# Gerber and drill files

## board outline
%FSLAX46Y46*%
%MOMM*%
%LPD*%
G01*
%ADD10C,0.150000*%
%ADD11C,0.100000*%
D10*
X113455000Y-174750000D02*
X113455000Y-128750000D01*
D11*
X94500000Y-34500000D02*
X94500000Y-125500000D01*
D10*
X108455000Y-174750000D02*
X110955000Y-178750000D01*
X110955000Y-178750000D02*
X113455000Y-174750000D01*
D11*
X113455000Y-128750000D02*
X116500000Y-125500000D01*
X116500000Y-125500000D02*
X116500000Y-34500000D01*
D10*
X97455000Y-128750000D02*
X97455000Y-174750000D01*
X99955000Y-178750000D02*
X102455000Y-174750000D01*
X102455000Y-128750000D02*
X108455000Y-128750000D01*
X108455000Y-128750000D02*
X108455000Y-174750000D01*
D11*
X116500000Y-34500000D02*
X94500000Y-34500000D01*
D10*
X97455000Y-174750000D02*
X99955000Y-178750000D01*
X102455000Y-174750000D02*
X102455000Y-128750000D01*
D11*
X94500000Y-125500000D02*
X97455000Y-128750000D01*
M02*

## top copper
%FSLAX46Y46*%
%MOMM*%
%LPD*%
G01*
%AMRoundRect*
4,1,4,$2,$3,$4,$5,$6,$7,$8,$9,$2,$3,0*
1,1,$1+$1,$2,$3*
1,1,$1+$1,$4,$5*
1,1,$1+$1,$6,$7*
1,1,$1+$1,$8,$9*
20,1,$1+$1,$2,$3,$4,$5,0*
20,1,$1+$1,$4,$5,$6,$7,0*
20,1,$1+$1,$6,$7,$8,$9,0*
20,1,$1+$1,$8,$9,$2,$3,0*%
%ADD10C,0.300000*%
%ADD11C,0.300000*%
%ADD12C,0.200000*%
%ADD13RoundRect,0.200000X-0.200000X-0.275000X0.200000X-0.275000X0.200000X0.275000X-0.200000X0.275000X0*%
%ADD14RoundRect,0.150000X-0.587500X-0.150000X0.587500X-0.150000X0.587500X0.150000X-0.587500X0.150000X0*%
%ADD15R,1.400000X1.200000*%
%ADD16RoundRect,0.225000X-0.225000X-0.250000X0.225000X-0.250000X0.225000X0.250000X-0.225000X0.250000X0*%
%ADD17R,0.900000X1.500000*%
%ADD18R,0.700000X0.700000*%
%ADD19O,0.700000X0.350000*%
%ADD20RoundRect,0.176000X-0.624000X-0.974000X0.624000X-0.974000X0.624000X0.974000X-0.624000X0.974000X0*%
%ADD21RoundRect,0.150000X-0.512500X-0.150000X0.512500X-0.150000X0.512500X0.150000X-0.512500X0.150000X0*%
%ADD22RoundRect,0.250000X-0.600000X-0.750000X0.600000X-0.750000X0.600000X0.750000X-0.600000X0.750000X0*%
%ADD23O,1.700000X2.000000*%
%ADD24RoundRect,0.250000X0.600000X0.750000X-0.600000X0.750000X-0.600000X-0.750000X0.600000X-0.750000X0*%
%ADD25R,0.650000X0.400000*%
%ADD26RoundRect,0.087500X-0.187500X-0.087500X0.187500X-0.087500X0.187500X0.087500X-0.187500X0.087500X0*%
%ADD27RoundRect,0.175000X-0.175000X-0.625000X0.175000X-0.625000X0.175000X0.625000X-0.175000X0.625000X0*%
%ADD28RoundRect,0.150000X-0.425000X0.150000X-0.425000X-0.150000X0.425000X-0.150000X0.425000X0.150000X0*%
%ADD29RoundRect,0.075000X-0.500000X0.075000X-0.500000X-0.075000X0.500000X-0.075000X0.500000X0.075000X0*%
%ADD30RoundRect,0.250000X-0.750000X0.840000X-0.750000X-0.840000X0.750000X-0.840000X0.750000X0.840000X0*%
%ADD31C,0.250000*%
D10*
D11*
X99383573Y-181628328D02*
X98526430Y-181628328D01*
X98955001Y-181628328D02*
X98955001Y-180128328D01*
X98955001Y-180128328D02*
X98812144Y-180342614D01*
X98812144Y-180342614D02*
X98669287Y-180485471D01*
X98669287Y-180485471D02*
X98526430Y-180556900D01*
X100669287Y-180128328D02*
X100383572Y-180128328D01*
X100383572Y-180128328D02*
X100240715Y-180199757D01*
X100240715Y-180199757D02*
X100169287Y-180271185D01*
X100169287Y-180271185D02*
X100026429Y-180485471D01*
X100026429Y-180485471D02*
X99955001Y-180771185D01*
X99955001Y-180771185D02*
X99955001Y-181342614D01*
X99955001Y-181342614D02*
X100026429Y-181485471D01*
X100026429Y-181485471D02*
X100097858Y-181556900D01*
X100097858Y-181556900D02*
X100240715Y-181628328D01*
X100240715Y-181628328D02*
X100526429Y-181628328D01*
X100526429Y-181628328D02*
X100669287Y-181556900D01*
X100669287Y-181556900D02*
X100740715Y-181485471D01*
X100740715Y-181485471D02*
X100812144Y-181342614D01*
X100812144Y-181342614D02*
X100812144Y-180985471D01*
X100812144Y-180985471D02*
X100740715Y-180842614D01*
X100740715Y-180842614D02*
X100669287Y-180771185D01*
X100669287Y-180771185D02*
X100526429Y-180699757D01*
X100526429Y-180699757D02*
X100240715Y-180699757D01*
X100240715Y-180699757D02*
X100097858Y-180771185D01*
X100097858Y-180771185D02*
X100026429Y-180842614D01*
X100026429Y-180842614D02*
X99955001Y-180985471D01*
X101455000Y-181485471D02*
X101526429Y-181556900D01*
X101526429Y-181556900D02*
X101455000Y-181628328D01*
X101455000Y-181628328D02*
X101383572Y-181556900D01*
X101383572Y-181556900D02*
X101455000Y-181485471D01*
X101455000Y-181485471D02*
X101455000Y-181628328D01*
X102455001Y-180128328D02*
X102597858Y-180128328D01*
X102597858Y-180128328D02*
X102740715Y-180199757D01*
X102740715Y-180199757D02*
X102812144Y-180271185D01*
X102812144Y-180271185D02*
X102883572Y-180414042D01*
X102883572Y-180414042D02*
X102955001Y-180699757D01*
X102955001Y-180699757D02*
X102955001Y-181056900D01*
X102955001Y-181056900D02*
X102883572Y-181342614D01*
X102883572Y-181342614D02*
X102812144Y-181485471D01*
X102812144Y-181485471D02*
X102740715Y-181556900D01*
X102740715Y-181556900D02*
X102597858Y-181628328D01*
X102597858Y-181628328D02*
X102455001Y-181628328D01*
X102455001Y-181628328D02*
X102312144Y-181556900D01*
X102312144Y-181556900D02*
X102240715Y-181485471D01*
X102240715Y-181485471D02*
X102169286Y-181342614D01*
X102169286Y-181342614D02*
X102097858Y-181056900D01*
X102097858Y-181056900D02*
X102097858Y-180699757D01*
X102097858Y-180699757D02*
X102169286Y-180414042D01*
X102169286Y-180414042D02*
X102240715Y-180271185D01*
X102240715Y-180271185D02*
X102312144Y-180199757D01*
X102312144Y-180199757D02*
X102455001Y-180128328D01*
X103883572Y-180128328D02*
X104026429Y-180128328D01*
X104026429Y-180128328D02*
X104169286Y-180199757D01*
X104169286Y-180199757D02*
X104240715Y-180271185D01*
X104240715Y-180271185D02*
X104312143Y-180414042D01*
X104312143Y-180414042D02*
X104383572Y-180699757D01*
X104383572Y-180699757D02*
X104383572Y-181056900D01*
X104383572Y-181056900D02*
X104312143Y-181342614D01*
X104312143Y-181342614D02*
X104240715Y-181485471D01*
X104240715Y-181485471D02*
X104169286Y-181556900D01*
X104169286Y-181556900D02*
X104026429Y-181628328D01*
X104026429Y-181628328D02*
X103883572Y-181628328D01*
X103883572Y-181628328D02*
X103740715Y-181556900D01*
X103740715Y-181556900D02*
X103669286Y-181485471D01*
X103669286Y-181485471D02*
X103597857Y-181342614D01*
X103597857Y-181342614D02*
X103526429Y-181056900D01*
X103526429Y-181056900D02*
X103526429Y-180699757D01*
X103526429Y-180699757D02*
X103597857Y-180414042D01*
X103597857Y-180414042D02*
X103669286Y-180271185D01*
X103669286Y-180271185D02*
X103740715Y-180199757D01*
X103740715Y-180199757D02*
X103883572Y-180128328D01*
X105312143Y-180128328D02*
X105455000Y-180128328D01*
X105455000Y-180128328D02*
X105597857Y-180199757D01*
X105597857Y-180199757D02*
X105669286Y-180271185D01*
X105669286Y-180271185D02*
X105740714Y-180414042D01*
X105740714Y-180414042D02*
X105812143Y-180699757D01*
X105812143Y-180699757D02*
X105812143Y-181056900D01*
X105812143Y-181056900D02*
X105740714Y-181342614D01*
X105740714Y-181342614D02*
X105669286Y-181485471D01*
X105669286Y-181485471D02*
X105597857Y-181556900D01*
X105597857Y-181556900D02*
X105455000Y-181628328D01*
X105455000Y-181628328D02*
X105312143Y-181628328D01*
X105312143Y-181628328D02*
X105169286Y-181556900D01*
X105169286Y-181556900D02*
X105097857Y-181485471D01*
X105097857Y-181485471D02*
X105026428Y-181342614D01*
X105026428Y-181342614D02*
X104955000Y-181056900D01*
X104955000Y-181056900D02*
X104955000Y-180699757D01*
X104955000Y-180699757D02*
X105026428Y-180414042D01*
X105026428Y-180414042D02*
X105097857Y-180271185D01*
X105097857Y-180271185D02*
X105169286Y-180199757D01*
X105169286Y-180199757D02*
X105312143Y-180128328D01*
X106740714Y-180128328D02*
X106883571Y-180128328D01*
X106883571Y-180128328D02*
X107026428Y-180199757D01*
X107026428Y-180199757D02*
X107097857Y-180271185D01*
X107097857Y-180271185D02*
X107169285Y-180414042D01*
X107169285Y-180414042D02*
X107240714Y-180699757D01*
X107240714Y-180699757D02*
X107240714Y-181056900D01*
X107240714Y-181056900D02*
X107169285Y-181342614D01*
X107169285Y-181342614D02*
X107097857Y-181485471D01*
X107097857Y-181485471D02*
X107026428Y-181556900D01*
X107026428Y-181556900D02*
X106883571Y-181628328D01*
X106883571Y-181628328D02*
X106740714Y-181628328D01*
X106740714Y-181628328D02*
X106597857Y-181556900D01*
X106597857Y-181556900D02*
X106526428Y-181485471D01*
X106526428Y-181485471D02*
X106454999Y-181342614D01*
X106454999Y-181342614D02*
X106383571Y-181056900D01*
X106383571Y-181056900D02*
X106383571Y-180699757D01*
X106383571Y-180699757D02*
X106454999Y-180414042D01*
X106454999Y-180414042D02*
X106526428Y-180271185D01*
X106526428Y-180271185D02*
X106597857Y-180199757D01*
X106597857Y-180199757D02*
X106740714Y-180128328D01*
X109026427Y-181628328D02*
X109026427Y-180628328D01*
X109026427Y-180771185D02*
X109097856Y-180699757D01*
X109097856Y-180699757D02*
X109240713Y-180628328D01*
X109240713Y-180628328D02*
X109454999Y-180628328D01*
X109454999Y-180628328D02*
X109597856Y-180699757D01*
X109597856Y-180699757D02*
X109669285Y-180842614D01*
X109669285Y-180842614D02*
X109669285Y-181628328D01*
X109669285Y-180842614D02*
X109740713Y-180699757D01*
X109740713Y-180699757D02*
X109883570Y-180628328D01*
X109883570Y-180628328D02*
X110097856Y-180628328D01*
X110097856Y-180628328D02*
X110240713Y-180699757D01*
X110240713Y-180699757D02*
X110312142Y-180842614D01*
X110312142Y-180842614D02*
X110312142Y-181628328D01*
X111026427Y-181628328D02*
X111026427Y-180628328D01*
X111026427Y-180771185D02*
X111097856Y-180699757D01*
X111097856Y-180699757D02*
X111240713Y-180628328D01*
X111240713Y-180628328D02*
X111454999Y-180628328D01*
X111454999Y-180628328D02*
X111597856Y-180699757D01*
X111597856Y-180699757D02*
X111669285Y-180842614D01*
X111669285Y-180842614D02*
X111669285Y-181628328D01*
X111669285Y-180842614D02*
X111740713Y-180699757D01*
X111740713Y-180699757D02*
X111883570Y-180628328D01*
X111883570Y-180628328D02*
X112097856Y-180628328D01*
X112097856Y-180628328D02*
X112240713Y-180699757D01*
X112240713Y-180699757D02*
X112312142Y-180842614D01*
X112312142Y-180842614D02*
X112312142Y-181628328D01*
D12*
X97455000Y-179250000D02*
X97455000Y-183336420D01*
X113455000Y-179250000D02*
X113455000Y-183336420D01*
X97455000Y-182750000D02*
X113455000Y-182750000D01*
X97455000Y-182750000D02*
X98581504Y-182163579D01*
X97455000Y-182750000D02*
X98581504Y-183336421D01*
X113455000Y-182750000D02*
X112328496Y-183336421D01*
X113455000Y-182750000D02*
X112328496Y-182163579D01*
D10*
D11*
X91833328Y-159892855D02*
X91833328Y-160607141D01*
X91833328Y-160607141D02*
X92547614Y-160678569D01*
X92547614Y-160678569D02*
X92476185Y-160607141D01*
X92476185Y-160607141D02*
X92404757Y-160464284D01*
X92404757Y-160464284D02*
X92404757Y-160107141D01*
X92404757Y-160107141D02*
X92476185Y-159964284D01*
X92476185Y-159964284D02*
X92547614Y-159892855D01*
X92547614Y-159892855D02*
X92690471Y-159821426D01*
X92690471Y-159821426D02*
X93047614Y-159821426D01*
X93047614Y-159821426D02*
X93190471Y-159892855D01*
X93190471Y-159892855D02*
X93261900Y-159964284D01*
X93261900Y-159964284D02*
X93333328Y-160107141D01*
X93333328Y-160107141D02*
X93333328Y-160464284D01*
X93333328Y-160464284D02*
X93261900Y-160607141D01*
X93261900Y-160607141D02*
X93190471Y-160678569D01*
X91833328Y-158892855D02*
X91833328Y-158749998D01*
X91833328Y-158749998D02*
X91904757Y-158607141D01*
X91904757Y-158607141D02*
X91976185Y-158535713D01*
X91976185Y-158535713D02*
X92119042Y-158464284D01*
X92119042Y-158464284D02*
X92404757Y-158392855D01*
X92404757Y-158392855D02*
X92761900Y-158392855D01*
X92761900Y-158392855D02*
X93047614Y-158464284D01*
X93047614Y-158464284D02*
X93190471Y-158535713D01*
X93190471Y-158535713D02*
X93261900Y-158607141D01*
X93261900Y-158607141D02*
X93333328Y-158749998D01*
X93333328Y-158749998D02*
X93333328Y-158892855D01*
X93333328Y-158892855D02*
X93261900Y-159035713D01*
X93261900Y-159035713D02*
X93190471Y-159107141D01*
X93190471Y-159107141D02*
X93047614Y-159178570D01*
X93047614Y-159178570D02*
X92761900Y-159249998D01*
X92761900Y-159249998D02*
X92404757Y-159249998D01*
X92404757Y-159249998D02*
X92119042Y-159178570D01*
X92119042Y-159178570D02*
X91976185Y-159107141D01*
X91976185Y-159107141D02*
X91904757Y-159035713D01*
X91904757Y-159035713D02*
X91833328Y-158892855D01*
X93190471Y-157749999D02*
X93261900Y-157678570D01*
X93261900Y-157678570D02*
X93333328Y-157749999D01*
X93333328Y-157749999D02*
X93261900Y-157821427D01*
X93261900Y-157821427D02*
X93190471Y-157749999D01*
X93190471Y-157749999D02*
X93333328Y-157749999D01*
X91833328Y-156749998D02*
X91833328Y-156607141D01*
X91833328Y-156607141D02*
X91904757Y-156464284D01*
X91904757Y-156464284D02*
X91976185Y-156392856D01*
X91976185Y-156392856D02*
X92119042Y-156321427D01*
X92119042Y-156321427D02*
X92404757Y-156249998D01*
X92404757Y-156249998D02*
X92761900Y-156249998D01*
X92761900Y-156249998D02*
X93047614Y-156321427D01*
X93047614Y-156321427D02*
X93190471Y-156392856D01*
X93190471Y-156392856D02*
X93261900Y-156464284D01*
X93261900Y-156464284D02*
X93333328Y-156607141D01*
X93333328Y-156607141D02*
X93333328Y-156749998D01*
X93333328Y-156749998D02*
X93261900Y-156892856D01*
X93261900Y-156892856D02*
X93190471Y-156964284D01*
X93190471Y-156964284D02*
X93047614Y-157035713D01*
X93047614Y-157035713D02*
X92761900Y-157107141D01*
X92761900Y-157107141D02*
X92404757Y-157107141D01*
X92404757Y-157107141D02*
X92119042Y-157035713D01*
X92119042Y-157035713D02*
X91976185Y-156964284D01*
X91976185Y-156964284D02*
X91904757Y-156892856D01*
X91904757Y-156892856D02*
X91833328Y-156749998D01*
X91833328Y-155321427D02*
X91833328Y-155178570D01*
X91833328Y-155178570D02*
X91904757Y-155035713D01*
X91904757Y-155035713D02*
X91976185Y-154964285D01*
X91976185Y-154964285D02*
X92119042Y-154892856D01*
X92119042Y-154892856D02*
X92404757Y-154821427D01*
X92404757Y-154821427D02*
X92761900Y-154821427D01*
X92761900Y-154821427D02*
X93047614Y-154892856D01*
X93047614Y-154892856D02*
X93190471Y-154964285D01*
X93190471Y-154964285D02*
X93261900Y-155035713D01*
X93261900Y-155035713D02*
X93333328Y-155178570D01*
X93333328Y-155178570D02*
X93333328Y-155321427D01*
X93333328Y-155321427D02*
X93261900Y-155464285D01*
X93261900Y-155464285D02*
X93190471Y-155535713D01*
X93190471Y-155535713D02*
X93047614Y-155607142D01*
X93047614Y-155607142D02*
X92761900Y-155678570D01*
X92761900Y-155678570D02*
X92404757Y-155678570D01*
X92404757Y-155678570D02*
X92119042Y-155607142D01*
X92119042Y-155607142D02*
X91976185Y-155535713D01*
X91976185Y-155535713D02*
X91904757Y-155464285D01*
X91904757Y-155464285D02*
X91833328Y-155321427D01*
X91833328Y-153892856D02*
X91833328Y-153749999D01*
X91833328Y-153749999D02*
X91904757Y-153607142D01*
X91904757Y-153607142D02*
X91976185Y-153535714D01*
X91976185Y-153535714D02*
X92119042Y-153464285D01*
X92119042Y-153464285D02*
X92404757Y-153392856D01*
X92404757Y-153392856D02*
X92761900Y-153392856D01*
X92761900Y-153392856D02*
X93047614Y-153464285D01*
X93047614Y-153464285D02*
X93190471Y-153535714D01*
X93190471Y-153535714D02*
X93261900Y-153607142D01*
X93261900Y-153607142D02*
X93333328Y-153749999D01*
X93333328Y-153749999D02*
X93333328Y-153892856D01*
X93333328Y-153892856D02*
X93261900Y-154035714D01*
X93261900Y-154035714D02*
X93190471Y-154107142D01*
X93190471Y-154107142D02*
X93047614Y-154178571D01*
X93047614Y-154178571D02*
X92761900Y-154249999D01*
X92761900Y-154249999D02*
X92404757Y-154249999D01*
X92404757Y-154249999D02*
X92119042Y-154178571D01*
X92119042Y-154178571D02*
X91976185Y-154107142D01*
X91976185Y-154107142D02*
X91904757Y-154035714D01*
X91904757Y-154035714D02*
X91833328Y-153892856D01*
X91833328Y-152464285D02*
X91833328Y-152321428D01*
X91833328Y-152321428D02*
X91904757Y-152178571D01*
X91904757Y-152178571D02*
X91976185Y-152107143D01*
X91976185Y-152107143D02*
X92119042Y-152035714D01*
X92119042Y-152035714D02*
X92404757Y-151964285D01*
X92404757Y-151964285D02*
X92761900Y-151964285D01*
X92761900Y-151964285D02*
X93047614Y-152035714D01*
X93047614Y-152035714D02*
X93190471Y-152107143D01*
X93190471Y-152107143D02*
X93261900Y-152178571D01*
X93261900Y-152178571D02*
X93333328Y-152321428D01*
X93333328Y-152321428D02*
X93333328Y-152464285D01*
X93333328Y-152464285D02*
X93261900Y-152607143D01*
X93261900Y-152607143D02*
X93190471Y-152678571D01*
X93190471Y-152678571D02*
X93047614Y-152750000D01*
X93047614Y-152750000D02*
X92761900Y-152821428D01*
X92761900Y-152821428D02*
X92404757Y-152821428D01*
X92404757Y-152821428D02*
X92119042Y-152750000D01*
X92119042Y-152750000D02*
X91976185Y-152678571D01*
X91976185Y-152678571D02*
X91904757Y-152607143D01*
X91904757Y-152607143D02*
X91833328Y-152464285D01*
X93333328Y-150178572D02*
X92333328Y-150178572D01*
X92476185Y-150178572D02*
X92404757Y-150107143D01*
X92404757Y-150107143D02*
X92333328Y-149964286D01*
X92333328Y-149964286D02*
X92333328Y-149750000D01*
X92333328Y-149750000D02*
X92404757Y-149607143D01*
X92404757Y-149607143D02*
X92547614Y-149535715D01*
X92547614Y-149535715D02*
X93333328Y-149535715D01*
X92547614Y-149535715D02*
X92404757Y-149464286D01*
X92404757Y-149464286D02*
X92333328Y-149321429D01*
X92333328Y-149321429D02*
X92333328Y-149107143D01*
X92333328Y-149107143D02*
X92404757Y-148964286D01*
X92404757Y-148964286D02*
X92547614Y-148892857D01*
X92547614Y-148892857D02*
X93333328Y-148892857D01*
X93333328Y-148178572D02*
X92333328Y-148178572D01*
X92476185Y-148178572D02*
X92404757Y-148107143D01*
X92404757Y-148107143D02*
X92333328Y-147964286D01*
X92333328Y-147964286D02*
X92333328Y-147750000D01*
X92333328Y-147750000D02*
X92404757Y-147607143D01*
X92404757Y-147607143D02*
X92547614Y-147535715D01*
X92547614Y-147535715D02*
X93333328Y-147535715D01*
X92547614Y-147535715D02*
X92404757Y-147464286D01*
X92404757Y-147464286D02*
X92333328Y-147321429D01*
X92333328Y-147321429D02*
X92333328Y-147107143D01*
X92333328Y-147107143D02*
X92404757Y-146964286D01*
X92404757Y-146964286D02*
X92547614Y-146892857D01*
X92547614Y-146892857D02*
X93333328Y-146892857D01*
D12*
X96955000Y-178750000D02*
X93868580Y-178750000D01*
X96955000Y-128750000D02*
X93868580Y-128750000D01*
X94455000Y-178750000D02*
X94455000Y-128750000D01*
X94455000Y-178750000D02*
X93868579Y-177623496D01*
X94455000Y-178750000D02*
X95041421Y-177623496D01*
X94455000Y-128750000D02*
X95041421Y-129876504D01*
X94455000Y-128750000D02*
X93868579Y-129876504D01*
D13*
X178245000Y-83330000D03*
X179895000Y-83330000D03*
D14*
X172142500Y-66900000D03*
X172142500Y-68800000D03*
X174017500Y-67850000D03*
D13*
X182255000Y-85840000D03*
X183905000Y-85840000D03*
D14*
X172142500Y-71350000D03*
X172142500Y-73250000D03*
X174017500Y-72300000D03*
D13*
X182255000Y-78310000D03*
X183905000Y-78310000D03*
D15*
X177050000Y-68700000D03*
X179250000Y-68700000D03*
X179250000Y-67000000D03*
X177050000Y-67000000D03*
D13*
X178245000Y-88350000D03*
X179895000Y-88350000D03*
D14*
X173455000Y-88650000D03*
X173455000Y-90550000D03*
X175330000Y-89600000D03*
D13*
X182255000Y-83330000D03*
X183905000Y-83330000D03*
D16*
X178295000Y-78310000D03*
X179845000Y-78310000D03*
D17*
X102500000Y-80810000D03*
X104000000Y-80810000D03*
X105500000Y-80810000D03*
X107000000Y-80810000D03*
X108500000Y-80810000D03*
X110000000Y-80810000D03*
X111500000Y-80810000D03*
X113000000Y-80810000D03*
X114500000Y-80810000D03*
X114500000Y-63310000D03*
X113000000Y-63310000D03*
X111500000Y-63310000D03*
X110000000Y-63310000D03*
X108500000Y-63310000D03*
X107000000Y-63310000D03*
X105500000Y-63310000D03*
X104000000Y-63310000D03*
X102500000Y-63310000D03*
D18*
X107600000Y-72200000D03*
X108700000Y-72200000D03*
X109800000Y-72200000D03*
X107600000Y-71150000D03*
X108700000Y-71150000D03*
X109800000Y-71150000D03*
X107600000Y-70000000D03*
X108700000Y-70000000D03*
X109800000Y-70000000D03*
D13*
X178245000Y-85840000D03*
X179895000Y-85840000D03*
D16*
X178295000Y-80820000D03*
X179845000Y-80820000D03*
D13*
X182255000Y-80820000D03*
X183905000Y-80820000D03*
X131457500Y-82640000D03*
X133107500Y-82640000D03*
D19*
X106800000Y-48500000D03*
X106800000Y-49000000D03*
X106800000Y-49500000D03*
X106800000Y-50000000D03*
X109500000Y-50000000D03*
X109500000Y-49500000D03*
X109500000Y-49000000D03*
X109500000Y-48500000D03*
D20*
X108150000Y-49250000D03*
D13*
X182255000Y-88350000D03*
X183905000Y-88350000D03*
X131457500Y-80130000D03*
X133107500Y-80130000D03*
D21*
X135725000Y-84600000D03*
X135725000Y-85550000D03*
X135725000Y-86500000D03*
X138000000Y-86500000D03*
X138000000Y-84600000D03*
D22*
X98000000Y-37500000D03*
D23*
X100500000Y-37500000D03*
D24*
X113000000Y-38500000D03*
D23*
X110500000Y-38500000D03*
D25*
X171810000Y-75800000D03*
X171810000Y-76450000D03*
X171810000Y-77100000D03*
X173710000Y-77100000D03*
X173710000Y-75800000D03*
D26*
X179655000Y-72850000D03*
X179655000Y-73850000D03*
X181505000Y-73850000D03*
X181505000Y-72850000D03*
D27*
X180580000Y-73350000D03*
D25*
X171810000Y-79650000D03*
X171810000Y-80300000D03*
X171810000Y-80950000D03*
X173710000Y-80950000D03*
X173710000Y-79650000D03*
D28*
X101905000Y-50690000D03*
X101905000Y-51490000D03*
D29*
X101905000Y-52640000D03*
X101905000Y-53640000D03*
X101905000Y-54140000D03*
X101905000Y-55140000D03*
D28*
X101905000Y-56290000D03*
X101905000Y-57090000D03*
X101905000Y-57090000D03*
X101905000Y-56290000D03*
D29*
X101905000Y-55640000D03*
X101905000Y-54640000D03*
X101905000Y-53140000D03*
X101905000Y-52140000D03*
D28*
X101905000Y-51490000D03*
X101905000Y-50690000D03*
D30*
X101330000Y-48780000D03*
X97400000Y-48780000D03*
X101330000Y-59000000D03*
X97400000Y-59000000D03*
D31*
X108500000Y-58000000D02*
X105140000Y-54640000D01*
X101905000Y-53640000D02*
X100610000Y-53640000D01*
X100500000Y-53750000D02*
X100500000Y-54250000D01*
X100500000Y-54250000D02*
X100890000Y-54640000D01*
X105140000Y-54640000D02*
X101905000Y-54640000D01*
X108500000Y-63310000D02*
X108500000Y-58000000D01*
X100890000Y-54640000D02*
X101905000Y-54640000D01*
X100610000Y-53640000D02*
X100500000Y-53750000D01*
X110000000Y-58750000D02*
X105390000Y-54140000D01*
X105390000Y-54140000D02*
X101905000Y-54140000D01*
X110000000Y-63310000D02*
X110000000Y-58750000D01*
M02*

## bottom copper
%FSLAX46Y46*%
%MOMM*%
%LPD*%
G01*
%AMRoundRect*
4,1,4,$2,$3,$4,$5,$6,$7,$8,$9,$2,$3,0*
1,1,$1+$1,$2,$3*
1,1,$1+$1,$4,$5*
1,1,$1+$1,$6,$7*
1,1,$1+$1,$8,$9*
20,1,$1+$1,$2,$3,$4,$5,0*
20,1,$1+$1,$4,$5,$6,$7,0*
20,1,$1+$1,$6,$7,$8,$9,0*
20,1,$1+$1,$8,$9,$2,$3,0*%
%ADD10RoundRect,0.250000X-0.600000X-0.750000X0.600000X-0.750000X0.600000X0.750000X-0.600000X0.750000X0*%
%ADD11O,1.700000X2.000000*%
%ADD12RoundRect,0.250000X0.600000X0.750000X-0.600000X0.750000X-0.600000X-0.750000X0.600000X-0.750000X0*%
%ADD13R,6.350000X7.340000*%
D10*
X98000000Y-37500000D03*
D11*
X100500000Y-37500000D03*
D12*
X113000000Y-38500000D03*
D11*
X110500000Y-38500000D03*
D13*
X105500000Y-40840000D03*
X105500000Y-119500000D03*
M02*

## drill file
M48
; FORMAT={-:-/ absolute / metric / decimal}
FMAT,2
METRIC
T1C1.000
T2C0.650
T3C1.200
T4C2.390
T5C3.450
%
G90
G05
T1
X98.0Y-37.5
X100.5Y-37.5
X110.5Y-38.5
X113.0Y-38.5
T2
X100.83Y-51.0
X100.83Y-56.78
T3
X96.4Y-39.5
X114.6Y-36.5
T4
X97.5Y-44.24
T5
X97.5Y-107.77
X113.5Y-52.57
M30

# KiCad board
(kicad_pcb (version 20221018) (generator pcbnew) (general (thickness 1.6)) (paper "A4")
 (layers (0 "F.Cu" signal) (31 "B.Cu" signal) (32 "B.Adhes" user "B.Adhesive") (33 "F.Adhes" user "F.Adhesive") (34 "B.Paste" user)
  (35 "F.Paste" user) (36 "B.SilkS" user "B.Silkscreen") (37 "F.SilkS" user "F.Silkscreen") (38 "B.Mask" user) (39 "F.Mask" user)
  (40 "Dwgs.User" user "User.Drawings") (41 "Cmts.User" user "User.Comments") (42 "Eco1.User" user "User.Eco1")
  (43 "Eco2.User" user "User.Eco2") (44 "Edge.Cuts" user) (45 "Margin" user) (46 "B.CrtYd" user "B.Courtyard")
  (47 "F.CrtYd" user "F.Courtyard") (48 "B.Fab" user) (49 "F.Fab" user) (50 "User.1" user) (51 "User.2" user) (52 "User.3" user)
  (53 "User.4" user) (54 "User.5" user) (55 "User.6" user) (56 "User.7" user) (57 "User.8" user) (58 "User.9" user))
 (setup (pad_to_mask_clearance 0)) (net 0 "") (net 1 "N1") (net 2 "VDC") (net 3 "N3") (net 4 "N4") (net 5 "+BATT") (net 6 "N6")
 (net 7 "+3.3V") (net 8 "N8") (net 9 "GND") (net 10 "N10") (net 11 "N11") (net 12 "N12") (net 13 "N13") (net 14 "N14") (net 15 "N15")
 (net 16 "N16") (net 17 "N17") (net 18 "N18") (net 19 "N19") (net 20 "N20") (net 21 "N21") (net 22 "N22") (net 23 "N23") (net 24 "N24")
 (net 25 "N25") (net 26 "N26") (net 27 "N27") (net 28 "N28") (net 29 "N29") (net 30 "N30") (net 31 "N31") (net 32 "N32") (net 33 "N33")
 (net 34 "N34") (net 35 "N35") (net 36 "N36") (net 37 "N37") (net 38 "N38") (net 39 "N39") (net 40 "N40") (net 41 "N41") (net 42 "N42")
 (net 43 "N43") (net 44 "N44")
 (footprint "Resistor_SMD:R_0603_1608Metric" (layer "F.Cu") (at 179.07 83.33)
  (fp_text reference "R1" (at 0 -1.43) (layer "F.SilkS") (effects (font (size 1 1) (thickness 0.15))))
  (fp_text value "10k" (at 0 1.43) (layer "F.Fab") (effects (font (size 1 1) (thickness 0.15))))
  (pad "1" smd roundrect (at -0.825 0) (size 0.8 0.95) (layers "F.Cu" "F.Paste" "F.Mask") (roundrect_rratio 0.25) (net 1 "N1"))
  (pad "2" smd roundrect (at 0.825 0) (size 0.8 0.95) (layers "F.Cu" "F.Paste" "F.Mask") (roundrect_rratio 0.25) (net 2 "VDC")))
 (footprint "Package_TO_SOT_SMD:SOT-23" (layer "F.Cu") (at 173.08 67.85)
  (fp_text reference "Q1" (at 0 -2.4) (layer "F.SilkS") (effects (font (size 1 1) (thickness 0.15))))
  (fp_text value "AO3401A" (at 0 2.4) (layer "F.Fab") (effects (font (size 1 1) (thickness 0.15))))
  (pad "1" smd roundrect (at -0.9375 -0.95) (size 1.475 0.6) (layers "F.Cu" "F.Paste" "F.Mask") (roundrect_rratio 0.25) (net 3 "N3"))
  (pad "2" smd roundrect (at -0.9375 0.95) (size 1.475 0.6) (layers "F.Cu" "F.Paste" "F.Mask") (roundrect_rratio 0.25) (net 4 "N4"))
  (pad "3" smd roundrect (at 0.9375 0) (size 1.475 0.6) (layers "F.Cu" "F.Paste" "F.Mask") (roundrect_rratio 0.25) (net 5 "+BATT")))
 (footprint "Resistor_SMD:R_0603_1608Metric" (layer "F.Cu") (at 183.08 85.84)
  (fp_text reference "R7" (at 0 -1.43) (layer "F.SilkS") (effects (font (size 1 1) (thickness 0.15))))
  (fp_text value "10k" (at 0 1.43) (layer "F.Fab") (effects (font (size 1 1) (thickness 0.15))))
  (pad "1" smd roundrect (at -0.825 0) (size 0.8 0.95) (layers "F.Cu" "F.Paste" "F.Mask") (roundrect_rratio 0.25) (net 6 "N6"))
  (pad "2" smd roundrect (at 0.825 0) (size 0.8 0.95) (layers "F.Cu" "F.Paste" "F.Mask") (roundrect_rratio 0.25) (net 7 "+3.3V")))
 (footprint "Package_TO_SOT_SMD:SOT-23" (layer "F.Cu") (at 173.08 72.3)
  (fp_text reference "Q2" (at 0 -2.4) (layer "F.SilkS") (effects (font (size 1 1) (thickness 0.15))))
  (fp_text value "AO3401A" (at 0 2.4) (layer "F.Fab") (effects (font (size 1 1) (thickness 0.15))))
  (pad "1" smd roundrect (at -0.9375 -0.95) (size 1.475 0.6) (layers "F.Cu" "F.Paste" "F.Mask") (roundrect_rratio 0.25) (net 6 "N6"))
  (pad "2" smd roundrect (at -0.9375 0.95) (size 1.475 0.6) (layers "F.Cu" "F.Paste" "F.Mask") (roundrect_rratio 0.25) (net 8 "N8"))
  (pad "3" smd roundrect (at 0.9375 0) (size 1.475 0.6) (layers "F.Cu" "F.Paste" "F.Mask") (roundrect_rratio 0.25) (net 7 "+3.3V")))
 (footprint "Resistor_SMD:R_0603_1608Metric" (layer "F.Cu") (at 183.08 78.31)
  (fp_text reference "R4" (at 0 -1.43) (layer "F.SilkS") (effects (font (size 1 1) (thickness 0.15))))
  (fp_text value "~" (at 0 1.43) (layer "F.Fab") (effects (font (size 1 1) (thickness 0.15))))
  (pad "1" smd roundrect (at -0.825 0) (size 0.8 0.95) (layers "F.Cu" "F.Paste" "F.Mask") (roundrect_rratio 0.25) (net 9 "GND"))
  (pad "2" smd roundrect (at 0.825 0) (size 0.8 0.95) (layers "F.Cu" "F.Paste" "F.Mask") (roundrect_rratio 0.25) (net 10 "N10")))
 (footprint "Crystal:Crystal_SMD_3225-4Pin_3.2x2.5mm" (layer "F.Cu") (at 178.15 67.85)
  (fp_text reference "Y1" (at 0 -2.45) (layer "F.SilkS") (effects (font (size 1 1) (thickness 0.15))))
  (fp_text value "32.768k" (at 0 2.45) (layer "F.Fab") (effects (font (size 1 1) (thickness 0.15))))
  (pad "1" smd rect (at -1.1 0.85) (size 1.4 1.2) (layers "F.Cu" "F.Paste" "F.Mask") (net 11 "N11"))
  (pad "2" smd rect (at 1.1 0.85) (size 1.4 1.2) (layers "F.Cu" "F.Paste" "F.Mask") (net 9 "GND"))
  (pad "3" smd rect (at 1.1 -0.85) (size 1.4 1.2) (layers "F.Cu" "F.Paste" "F.Mask") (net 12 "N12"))
  (pad "4" smd rect (at -1.1 -0.85) (size 1.4 1.2) (layers "F.Cu" "F.Paste" "F.Mask") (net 9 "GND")))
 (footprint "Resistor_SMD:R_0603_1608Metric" (layer "F.Cu") (at 179.07 88.35)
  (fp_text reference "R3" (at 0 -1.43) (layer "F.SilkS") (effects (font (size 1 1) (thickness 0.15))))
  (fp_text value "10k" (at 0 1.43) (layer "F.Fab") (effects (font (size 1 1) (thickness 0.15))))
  (pad "1" smd roundrect (at -0.825 0) (size 0.8 0.95) (layers "F.Cu" "F.Paste" "F.Mask") (roundrect_rratio 0.25) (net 7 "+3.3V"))
  (pad "2" smd roundrect (at 0.825 0) (size 0.8 0.95) (layers "F.Cu" "F.Paste" "F.Mask") (roundrect_rratio 0.25) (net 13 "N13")))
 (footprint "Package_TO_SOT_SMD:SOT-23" (layer "F.Cu") (at 174.3925 89.6)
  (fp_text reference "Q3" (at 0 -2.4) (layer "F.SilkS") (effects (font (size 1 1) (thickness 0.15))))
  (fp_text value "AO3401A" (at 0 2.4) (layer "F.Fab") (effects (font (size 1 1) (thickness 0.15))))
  (pad "1" smd roundrect (at -0.9375 -0.95) (size 1.475 0.6) (layers "F.Cu" "F.Paste" "F.Mask") (roundrect_rratio 0.25) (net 2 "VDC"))
  (pad "2" smd roundrect (at -0.9375 0.95) (size 1.475 0.6) (layers "F.Cu" "F.Paste" "F.Mask") (roundrect_rratio 0.25) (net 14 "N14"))
  (pad "3" smd roundrect (at 0.9375 0) (size 1.475 0.6) (layers "F.Cu" "F.Paste" "F.Mask") (roundrect_rratio 0.25) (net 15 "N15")))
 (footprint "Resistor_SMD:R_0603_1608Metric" (layer "F.Cu") (at 183.08 83.33)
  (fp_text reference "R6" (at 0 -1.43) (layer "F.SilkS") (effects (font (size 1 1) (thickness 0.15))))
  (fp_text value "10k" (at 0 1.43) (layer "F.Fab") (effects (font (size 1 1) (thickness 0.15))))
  (pad "1" smd roundrect (at -0.825 0) (size 0.8 0.95) (layers "F.Cu" "F.Paste" "F.Mask") (roundrect_rratio 0.25) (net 7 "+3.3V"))
  (pad "2" smd roundrect (at 0.825 0) (size 0.8 0.95) (layers "F.Cu" "F.Paste" "F.Mask") (roundrect_rratio 0.25) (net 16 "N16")))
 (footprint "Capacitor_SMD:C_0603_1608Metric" (layer "F.Cu") (at 179.07 78.31)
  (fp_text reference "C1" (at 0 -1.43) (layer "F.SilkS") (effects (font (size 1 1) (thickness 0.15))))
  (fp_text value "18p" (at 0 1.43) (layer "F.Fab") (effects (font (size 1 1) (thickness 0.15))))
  (pad "1" smd roundrect (at -0.775 0) (size 0.9 0.95) (layers "F.Cu" "F.Paste" "F.Mask") (roundrect_rratio 0.25) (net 11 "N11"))
  (pad "2" smd roundrect (at 0.775 0) (size 0.9 0.95) (layers "F.Cu" "F.Paste" "F.Mask") (roundrect_rratio 0.25) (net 9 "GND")))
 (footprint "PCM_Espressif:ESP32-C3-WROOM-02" (layer "F.Cu") (at 108.4 72.06 90)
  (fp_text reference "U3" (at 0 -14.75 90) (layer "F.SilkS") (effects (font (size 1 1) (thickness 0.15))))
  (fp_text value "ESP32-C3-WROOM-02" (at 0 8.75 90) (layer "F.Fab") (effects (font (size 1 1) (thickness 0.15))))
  (pad "1" smd rect (at -8.75 -5.9 90) (size 1.5 0.9) (layers "F.Cu" "F.Paste" "F.Mask") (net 7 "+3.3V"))
  (pad "2" smd rect (at -8.75 -4.4 90) (size 1.5 0.9) (layers "F.Cu" "F.Paste" "F.Mask") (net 13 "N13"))
  (pad "3" smd rect (at -8.75 -2.9 90) (size 1.5 0.9) (layers "F.Cu" "F.Paste" "F.Mask") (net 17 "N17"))
  (pad "4" smd rect (at -8.75 -1.4 90) (size 1.5 0.9) (layers "F.Cu" "F.Paste" "F.Mask") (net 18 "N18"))
  (pad "5" smd rect (at -8.75 0.1 90) (size 1.5 0.9) (layers "F.Cu" "F.Paste" "F.Mask") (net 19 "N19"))
  (pad "6" smd rect (at -8.75 1.6 90) (size 1.5 0.9) (layers "F.Cu" "F.Paste" "F.Mask") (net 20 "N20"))
  (pad "7" smd rect (at -8.75 3.1 90) (size 1.5 0.9) (layers "F.Cu" "F.Paste" "F.Mask") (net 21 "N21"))
  (pad "8" smd rect (at -8.75 4.6 90) (size 1.5 0.9) (layers "F.Cu" "F.Paste" "F.Mask") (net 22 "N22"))
  (pad "9" smd rect (at -8.75 6.1 90) (size 1.5 0.9) (layers "F.Cu" "F.Paste" "F.Mask") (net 9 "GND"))
  (pad "10" smd rect (at 8.75 6.1 270) (size 1.5 0.9) (layers "F.Cu" "F.Paste" "F.Mask") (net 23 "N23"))
  (pad "11" smd rect (at 8.75 4.6 270) (size 1.5 0.9) (layers "F.Cu" "F.Paste" "F.Mask") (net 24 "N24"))
  (pad "12" smd rect (at 8.75 3.1 270) (size 1.5 0.9) (layers "F.Cu" "F.Paste" "F.Mask") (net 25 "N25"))
  (pad "13" smd rect (at 8.75 1.6 270) (size 1.5 0.9) (layers "F.Cu" "F.Paste" "F.Mask") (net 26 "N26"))
  (pad "14" smd rect (at 8.75 0.1 270) (size 1.5 0.9) (layers "F.Cu" "F.Paste" "F.Mask") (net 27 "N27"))
  (pad "15" smd rect (at 8.75 -1.4 270) (size 1.5 0.9) (layers "F.Cu" "F.Paste" "F.Mask") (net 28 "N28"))
  (pad "16" smd rect (at 8.75 -2.9 270) (size 1.5 0.9) (layers "F.Cu" "F.Paste" "F.Mask") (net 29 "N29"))
  (pad "17" smd rect (at 8.75 -4.4 270) (size 1.5 0.9) (layers "F.Cu" "F.Paste" "F.Mask") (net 12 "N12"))
  (pad "18" smd rect (at 8.75 -5.9 270) (size 1.5 0.9) (layers "F.Cu" "F.Paste" "F.Mask") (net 11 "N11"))
  (pad "19" smd rect (at -0.14 -0.8 270) (size 0.7 0.7) (layers "F.Cu" "F.Paste" "F.Mask") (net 9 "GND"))
  (pad "19" smd rect (at -0.14 0.3 270) (size 0.7 0.7) (layers "F.Cu" "F.Paste" "F.Mask") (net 9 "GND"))
  (pad "19" smd rect (at -0.14 1.4 270) (size 0.7 0.7) (layers "F.Cu" "F.Paste" "F.Mask") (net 9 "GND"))
  (pad "19" smd rect (at 0.91 -0.8 270) (size 0.7 0.7) (layers "F.Cu" "F.Paste" "F.Mask") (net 9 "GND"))
  (pad "19" smd rect (at 0.91 0.3 270) (size 0.7 0.7) (layers "F.Cu" "F.Paste" "F.Mask") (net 9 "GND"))
  (pad "19" smd rect (at 0.91 1.4 270) (size 0.7 0.7) (layers "F.Cu" "F.Paste" "F.Mask") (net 9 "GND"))
  (pad "19" smd rect (at 2.06 -0.8 270) (size 0.7 0.7) (layers "F.Cu" "F.Paste" "F.Mask") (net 9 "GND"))
  (pad "19" smd rect (at 2.06 0.3 270) (size 0.7 0.7) (layers "F.Cu" "F.Paste" "F.Mask") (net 9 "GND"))
  (pad "19" smd rect (at 2.06 1.4 270) (size 0.7 0.7) (layers "F.Cu" "F.Paste" "F.Mask") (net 9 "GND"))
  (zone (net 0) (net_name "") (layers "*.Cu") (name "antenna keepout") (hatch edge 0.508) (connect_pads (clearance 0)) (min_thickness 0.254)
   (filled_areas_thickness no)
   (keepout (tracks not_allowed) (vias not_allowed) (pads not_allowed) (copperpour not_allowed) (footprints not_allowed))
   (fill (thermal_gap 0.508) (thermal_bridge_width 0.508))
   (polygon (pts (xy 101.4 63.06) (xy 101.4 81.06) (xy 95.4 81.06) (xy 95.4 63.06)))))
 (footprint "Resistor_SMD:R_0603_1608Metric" (layer "F.Cu") (at 179.07 85.84)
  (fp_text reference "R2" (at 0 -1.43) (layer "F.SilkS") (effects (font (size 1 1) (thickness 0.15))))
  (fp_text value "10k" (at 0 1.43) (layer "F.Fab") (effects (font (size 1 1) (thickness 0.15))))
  (pad "1" smd roundrect (at -0.825 0) (size 0.8 0.95) (layers "F.Cu" "F.Paste" "F.Mask") (roundrect_rratio 0.25) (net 2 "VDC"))
  (pad "2" smd roundrect (at 0.825 0) (size 0.8 0.95) (layers "F.Cu" "F.Paste" "F.Mask") (roundrect_rratio 0.25) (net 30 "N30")))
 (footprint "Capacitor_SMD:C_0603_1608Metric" (layer "F.Cu") (at 179.07 80.82)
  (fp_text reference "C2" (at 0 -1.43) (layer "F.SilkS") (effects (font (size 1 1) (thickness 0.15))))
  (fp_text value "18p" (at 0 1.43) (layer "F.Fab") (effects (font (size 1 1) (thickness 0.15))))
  (pad "1" smd roundrect (at -0.775 0) (size 0.9 0.95) (layers "F.Cu" "F.Paste" "F.Mask") (roundrect_rratio 0.25) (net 12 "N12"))
  (pad "2" smd roundrect (at 0.775 0) (size 0.9 0.95) (layers "F.Cu" "F.Paste" "F.Mask") (roundrect_rratio 0.25) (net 9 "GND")))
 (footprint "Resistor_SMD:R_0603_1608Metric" (layer "F.Cu") (at 183.08 80.82)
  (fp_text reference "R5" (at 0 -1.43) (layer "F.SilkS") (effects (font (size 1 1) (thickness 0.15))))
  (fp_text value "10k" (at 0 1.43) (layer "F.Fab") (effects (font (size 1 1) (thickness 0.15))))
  (pad "1" smd roundrect (at -0.825 0) (size 0.8 0.95) (layers "F.Cu" "F.Paste" "F.Mask") (roundrect_rratio 0.25) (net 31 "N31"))
  (pad "2" smd roundrect (at 0.825 0) (size 0.8 0.95) (layers "F.Cu" "F.Paste" "F.Mask") (roundrect_rratio 0.25) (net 7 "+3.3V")))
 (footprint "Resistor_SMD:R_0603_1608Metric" (layer "F.Cu") (at 132.2825 82.64)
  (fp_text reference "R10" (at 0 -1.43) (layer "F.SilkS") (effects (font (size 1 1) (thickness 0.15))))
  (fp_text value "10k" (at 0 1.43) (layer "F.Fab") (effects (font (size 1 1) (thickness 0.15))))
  (pad "1" smd roundrect (at -0.825 0) (size 0.8 0.95) (layers "F.Cu" "F.Paste" "F.Mask") (roundrect_rratio 0.25) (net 9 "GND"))
  (pad "2" smd roundrect (at 0.825 0) (size 0.8 0.95) (layers "F.Cu" "F.Paste" "F.Mask") (roundrect_rratio 0.25) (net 2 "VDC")))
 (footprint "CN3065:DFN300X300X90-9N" (layer "F.Cu") (at 108.15 49.25)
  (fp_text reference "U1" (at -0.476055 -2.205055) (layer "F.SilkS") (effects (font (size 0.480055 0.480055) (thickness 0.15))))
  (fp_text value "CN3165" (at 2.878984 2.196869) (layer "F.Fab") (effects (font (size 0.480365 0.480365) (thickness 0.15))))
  (pad "1" smd oval (at -1.35 -0.75) (size 0.7 0.35) (layers "F.Cu" "F.Paste") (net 9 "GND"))
  (pad "2" smd oval (at -1.35 -0.25) (size 0.7 0.35) (layers "F.Cu" "F.Paste") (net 10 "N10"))
  (pad "3" smd oval (at -1.35 0.25) (size 0.7 0.35) (layers "F.Cu" "F.Paste") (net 9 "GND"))
  (pad "4" smd oval (at -1.35 0.75) (size 0.7 0.35) (layers "F.Cu" "F.Paste") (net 14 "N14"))
  (pad "5" smd oval (at 1.35 0.75) (size 0.7 0.35) (layers "F.Cu" "F.Paste") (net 5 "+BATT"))
  (pad "6" smd oval (at 1.35 0.25) (size 0.7 0.35) (layers "F.Cu" "F.Paste") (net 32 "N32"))
  (pad "7" smd oval (at 1.35 -0.25) (size 0.7 0.35) (layers "F.Cu" "F.Paste") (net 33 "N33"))
  (pad "8" smd oval (at 1.35 -0.75) (size 0.7 0.35) (layers "F.Cu" "F.Paste") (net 5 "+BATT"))
  (pad "9" smd roundrect (at 0 0) (size 1.6 2.3) (layers "F.Cu" "F.Mask") (roundrect_rratio 0.11) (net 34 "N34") (solder_mask_margin 0.102)))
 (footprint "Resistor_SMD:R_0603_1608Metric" (layer "F.Cu") (at 183.08 88.35)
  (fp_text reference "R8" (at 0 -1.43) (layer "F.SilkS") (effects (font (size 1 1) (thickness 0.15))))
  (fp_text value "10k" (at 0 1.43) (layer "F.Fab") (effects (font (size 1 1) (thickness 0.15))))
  (pad "1" smd roundrect (at -0.825 0) (size 0.8 0.95) (layers "F.Cu" "F.Paste" "F.Mask") (roundrect_rratio 0.25) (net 3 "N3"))
  (pad "2" smd roundrect (at 0.825 0) (size 0.8 0.95) (layers "F.Cu" "F.Paste" "F.Mask") (roundrect_rratio 0.25) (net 5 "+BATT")))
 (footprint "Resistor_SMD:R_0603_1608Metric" (layer "F.Cu") (at 132.2825 80.13)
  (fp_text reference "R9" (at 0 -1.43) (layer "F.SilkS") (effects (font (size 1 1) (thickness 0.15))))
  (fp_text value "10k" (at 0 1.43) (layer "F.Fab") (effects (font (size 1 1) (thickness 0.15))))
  (pad "1" smd roundrect (at -0.825 0) (size 0.8 0.95) (layers "F.Cu" "F.Paste" "F.Mask") (roundrect_rratio 0.25) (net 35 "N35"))
  (pad "2" smd roundrect (at 0.825 0) (size 0.8 0.95) (layers "F.Cu" "F.Paste" "F.Mask") (roundrect_rratio 0.25) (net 2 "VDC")))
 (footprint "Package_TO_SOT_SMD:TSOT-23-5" (layer "F.Cu") (at 136.8625 85.55)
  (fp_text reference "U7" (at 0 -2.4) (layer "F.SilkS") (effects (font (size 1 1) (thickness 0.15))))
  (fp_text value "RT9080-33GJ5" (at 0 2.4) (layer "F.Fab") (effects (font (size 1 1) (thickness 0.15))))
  (pad "1" smd roundrect (at -1.1375 -0.95) (size 1.325 0.6) (layers "F.Cu" "F.Paste" "F.Mask") (roundrect_rratio 0.25) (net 5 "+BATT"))
  (pad "2" smd roundrect (at -1.1375 0) (size 1.325 0.6) (layers "F.Cu" "F.Paste" "F.Mask") (roundrect_rratio 0.25) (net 9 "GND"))
  (pad "3" smd roundrect (at -1.1375 0.95) (size 1.325 0.6) (layers "F.Cu" "F.Paste" "F.Mask") (roundrect_rratio 0.25) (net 5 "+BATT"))
  (pad "4" smd roundrect (at 1.1375 0.95) (size 1.325 0.6) (layers "F.Cu" "F.Paste" "F.Mask") (roundrect_rratio 0.25) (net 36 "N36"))
  (pad "5" smd roundrect (at 1.1375 -0.95) (size 1.325 0.6) (layers "F.Cu" "F.Paste" "F.Mask") (roundrect_rratio 0.25) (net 7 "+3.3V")))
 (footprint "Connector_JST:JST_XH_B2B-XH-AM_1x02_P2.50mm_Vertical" (layer "F.Cu") (at 98 37.5)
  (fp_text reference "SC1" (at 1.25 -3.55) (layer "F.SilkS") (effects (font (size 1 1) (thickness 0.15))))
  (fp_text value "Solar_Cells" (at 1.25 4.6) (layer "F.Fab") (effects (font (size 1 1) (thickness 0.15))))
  (pad "" np_thru_hole circle (at -1.6 2) (size 1.2 1.2) (drill 1.2) (layers "*.Cu" "*.Mask"))
  (pad "1" thru_hole roundrect (at 0 0) (size 1.7 2) (drill 1) (layers "*.Cu" "*.Mask") (roundrect_rratio 0.147059) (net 15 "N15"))
  (pad "2" thru_hole oval (at 2.5 0) (size 1.7 2) (drill 1) (layers "*.Cu" "*.Mask") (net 9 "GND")))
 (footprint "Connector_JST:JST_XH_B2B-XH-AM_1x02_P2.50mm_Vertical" (layer "F.Cu") (at 113 38.5 180)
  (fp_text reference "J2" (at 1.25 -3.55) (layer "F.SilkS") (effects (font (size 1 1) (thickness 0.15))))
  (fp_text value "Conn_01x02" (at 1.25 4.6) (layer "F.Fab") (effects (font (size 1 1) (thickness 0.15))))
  (pad "" np_thru_hole circle (at -1.6 2 180) (size 1.2 1.2) (drill 1.2) (layers "*.Cu" "*.Mask"))
  (pad "1" thru_hole roundrect (at 0 0 180) (size 1.7 2) (drill 1) (layers "*.Cu" "*.Mask") (roundrect_rratio 0.147059) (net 4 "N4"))
  (pad "2" thru_hole oval (at 2.5 0 180) (size 1.7 2) (drill 1) (layers "*.Cu" "*.Mask") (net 9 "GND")))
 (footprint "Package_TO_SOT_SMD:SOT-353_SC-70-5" (layer "F.Cu") (at 172.76 76.45)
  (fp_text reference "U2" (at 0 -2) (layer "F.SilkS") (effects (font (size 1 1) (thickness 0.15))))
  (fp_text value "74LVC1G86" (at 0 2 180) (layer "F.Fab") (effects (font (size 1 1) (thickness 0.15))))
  (pad "1" smd rect (at -0.95 -0.65) (size 0.65 0.4) (layers "F.Cu" "F.Paste" "F.Mask") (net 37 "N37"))
  (pad "2" smd rect (at -0.95 0) (size 0.65 0.4) (layers "F.Cu" "F.Paste" "F.Mask") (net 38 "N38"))
  (pad "3" smd rect (at -0.95 0.65) (size 0.65 0.4) (layers "F.Cu" "F.Paste" "F.Mask") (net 9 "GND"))
  (pad "4" smd rect (at 0.95 0.65) (size 0.65 0.4) (layers "F.Cu" "F.Paste" "F.Mask") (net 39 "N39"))
  (pad "5" smd rect (at 0.95 -0.65) (size 0.65 0.4) (layers "F.Cu" "F.Paste" "F.Mask") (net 8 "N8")))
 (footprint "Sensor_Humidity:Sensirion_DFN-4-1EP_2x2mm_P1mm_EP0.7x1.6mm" (layer "F.Cu") (at 180.58 73.35)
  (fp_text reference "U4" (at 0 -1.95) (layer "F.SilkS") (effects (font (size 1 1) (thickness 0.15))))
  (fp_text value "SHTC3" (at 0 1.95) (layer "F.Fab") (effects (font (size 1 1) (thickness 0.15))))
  (pad "" smd roundrect (at -1.025 -0.5) (size 0.55 0.35) (layers "F.Paste") (roundrect_rratio 0.25))
  (pad "" smd roundrect (at -1.025 0.5) (size 0.55 0.35) (layers "F.Paste") (roundrect_rratio 0.25))
  (pad "" smd roundrect (at 0 0) (size 0.5 1.4) (layers "F.Paste") (roundrect_rratio 0.25))
  (pad "" smd roundrect (at 1.025 -0.5 180) (size 0.55 0.35) (layers "F.Paste") (roundrect_rratio 0.25))
  (pad "" smd roundrect (at 1.025 0.5 180) (size 0.55 0.35) (layers "F.Paste") (roundrect_rratio 0.25))
  (pad "1" smd roundrect (at -0.925 -0.5) (size 0.55 0.35) (layers "F.Cu" "F.Mask") (roundrect_rratio 0.25) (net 7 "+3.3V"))
  (pad "2" smd roundrect (at -0.925 0.5) (size 0.55 0.35) (layers "F.Cu" "F.Mask") (roundrect_rratio 0.25) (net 16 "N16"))
  (pad "3" smd roundrect (at 0.925 0.5) (size 0.55 0.35) (layers "F.Cu" "F.Mask") (roundrect_rratio 0.25) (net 31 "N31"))
  (pad "4" smd roundrect (at 0.925 -0.5) (size 0.55 0.35) (layers "F.Cu" "F.Mask") (roundrect_rratio 0.25) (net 9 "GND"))
  (pad "5" smd roundrect (at 0 0) (size 0.7 1.6) (layers "F.Cu" "F.Mask") (roundrect_rratio 0.25) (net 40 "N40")))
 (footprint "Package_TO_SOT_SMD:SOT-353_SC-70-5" (layer "F.Cu") (at 172.76 80.3)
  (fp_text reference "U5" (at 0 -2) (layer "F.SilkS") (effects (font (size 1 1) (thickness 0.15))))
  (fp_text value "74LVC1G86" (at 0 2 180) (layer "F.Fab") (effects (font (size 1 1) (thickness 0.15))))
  (pad "1" smd rect (at -0.95 -0.65) (size 0.65 0.4) (layers "F.Cu" "F.Paste" "F.Mask") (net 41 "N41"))
  (pad "2" smd rect (at -0.95 0) (size 0.65 0.4) (layers "F.Cu" "F.Paste" "F.Mask") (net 9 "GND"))
  (pad "3" smd rect (at -0.95 0.65) (size 0.65 0.4) (layers "F.Cu" "F.Paste" "F.Mask") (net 9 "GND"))
  (pad "4" smd rect (at 0.95 0.65) (size 0.65 0.4) (layers "F.Cu" "F.Paste" "F.Mask") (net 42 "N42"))
  (pad "5" smd rect (at 0.95 -0.65) (size 0.65 0.4) (layers "F.Cu" "F.Paste" "F.Mask") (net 8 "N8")))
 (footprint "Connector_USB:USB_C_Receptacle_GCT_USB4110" (layer "F.Cu") (at 98.225 53.89 -90)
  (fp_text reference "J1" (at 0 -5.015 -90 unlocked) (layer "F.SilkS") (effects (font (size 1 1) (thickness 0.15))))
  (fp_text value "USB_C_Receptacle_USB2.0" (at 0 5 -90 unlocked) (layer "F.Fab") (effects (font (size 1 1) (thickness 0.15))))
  (pad "" np_thru_hole circle (at -2.89 -2.605 270) (size 0.65 0.65) (drill 0.65) (layers "F&B.Cu" "*.Mask"))
  (pad "" np_thru_hole circle (at 2.89 -2.605 270) (size 0.65 0.65) (drill 0.65) (layers "F&B.Cu" "*.Mask"))
  (pad "A1" smd roundrect (at -3.2 -3.68 270) (size 0.6 1.15) (layers "F.Cu" "F.Paste" "F.Mask") (roundrect_rratio 0.25) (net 9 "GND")
   (thermal_bridge_angle 45))
  (pad "A4" smd roundrect (at -2.4 -3.68 270) (size 0.6 1.15) (layers "F.Cu" "F.Paste" "F.Mask") (roundrect_rratio 0.25) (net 2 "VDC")
   (thermal_bridge_angle 45))
  (pad "A5" smd roundrect (at -1.25 -3.68 270) (size 0.3 1.15) (layers "F.Cu" "F.Paste" "F.Mask") (roundrect_rratio 0.25) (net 30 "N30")
   (thermal_bridge_angle 45))
  (pad "A6" smd roundrect (at -0.25 -3.68 270) (size 0.3 1.15) (layers "F.Cu" "F.Paste" "F.Mask") (roundrect_rratio 0.25) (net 27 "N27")
   (thermal_bridge_angle 45))
  (pad "A7" smd roundrect (at 0.25 -3.68 270) (size 0.3 1.15) (layers "F.Cu" "F.Paste" "F.Mask") (roundrect_rratio 0.25) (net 26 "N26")
   (thermal_bridge_angle 45))
  (pad "A8" smd roundrect (at 1.25 -3.68 270) (size 0.3 1.15) (layers "F.Cu" "F.Paste" "F.Mask") (roundrect_rratio 0.25) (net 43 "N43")
   (thermal_bridge_angle 45))
  (pad "A9" smd roundrect (at 2.4 -3.68 270) (size 0.6 1.15) (layers "F.Cu" "F.Paste" "F.Mask") (roundrect_rratio 0.25) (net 2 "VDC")
   (thermal_bridge_angle 45))
  (pad "A12" smd roundrect (at 3.2 -3.68 270) (size 0.6 1.15) (layers "F.Cu" "F.Paste" "F.Mask") (roundrect_rratio 0.25) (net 9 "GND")
   (thermal_bridge_angle 45))
  (pad "B1" smd roundrect (at 3.2 -3.68 270) (size 0.6 1.15) (layers "F.Cu" "F.Paste" "F.Mask") (roundrect_rratio 0.25) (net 9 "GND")
   (thermal_bridge_angle 45))
  (pad "B4" smd roundrect (at 2.4 -3.68 270) (size 0.6 1.15) (layers "F.Cu" "F.Paste" "F.Mask") (roundrect_rratio 0.25) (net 2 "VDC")
   (thermal_bridge_angle 45))
  (pad "B5" smd roundrect (at 1.75 -3.68 270) (size 0.3 1.15) (layers "F.Cu" "F.Paste" "F.Mask") (roundrect_rratio 0.25) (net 1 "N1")
   (thermal_bridge_angle 45))
  (pad "B6" smd roundrect (at 0.75 -3.68 270) (size 0.3 1.15) (layers "F.Cu" "F.Paste" "F.Mask") (roundrect_rratio 0.25) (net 27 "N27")
   (thermal_bridge_angle 45))
  (pad "B7" smd roundrect (at -0.75 -3.68 270) (size 0.3 1.15) (layers "F.Cu" "F.Paste" "F.Mask") (roundrect_rratio 0.25) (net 26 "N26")
   (thermal_bridge_angle 45))
  (pad "B8" smd roundrect (at -1.75 -3.68 270) (size 0.3 1.15) (layers "F.Cu" "F.Paste" "F.Mask") (roundrect_rratio 0.25) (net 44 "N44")
   (thermal_bridge_angle 45))
  (pad "B9" smd roundrect (at -2.4 -3.68 270) (size 0.6 1.15) (layers "F.Cu" "F.Paste" "F.Mask") (roundrect_rratio 0.25) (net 2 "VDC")
   (thermal_bridge_angle 45))
  (pad "B12" smd roundrect (at -3.2 -3.68 270) (size 0.6 1.15) (layers "F.Cu" "F.Paste" "F.Mask") (roundrect_rratio 0.25) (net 9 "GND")
   (thermal_bridge_angle 45))
  (pad "S1" smd roundrect (at -5.11 -3.105 270) (size 2.18 2) (layers "F.Cu" "F.Paste" "F.Mask") (roundrect_rratio 0.125) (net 9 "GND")
   (thermal_bridge_angle 45))
  (pad "S1" smd roundrect (at -5.11 0.825 270) (size 2.18 2) (layers "F.Cu" "F.Paste" "F.Mask") (roundrect_rratio 0.125) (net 9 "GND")
   (thermal_bridge_angle 45))
  (pad "S1" smd roundrect (at 5.11 -3.105 270) (size 2.18 2) (layers "F.Cu" "F.Paste" "F.Mask") (roundrect_rratio 0.125) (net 9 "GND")
   (thermal_bridge_angle 45))
  (pad "S1" smd roundrect (at 5.11 0.825 270) (size 2.18 2) (layers "F.Cu" "F.Paste" "F.Mask") (roundrect_rratio 0.125) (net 9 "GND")
   (thermal_bridge_angle 45)))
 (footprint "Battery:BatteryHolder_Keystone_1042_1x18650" (layer "B.Cu") (at 105.5 80.17 -90)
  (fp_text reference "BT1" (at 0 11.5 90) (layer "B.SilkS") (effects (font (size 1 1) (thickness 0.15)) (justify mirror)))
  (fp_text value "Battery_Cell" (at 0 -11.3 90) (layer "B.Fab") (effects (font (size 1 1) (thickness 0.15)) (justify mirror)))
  (pad "" np_thru_hole circle (at -35.93 8 270) (size 2.39 2.39) (drill 2.39) (layers "*.Cu" "*.Mask"))
  (pad "" np_thru_hole circle (at -27.6 -8 270) (size 3.45 3.45) (drill 3.45) (layers "*.Cu" "*.Mask"))
  (pad "" np_thru_hole circle (at 27.6 8 270) (size 3.45 3.45) (drill 3.45) (layers "*.Cu" "*.Mask"))
  (pad "1" smd rect (at -39.33 0 270) (size 7.34 6.35) (layers "B.Cu" "B.Paste" "B.Mask") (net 5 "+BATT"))
  (pad "2" smd rect (at 39.33 0 270) (size 7.34 6.35) (layers "B.Cu" "B.Paste" "B.Mask") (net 9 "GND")))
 (gr_line (start 113.455 174.75) (end 113.455 128.75) (stroke (width 0.15) (type default)) (layer "Edge.Cuts"))
 (gr_line (start 94.5 34.5) (end 94.5 125.5) (stroke (width 0.1) (type default)) (layer "Edge.Cuts"))
 (gr_line (start 108.455 174.75) (end 110.955 178.75) (stroke (width 0.15) (type default)) (layer "Edge.Cuts"))
 (gr_line (start 110.955 178.75) (end 113.455 174.75) (stroke (width 0.15) (type default)) (layer "Edge.Cuts"))
 (gr_line (start 113.455 128.75) (end 116.5 125.5) (stroke (width 0.1) (type default)) (layer "Edge.Cuts"))
 (gr_line (start 116.5 125.5) (end 116.5 34.5) (stroke (width 0.1) (type default)) (layer "Edge.Cuts"))
 (gr_line (start 97.455 128.75) (end 97.455 174.75) (stroke (width 0.15) (type default)) (layer "Edge.Cuts"))
 (gr_line (start 99.955 178.75) (end 102.455 174.75) (stroke (width 0.15) (type default)) (layer "Edge.Cuts"))
 (gr_line (start 102.455 128.75) (end 108.455 128.75) (stroke (width 0.15) (type default)) (layer "Edge.Cuts"))
 (gr_line (start 108.455 128.75) (end 108.455 174.75) (stroke (width 0.15) (type default)) (layer "Edge.Cuts"))
 (gr_line (start 116.5 34.5) (end 94.5 34.5) (stroke (width 0.1) (type default)) (layer "Edge.Cuts"))
 (gr_line (start 97.455 174.75) (end 99.955 178.75) (stroke (width 0.15) (type default)) (layer "Edge.Cuts"))
 (gr_line (start 102.455 174.75) (end 102.455 128.75) (stroke (width 0.15) (type default)) (layer "Edge.Cuts"))
 (gr_line (start 94.5 125.5) (end 97.455 128.75) (stroke (width 0.1) (type default)) (layer "Edge.Cuts"))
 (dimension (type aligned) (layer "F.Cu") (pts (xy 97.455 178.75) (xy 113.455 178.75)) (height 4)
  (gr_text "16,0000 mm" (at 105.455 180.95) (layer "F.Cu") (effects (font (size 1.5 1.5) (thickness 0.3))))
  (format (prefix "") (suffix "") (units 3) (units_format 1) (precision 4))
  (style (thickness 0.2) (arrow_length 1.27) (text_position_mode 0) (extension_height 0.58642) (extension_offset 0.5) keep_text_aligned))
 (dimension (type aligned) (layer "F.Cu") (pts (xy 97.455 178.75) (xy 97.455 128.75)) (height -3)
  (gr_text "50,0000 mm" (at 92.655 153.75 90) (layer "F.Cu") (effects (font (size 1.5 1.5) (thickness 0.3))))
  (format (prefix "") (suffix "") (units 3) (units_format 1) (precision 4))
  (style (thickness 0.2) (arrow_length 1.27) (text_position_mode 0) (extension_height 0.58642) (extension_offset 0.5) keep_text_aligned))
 (segment (start 108.5 58) (end 105.14 54.64) (width 0.25) (layer "F.Cu") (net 27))
 (segment (start 101.905 53.64) (end 100.61 53.64) (width 0.25) (layer "F.Cu") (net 27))
 (segment (start 100.5 53.75) (end 100.5 54.25) (width 0.25) (layer "F.Cu") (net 27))
 (segment (start 100.5 54.25) (end 100.89 54.64) (width 0.25) (layer "F.Cu") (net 27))
 (segment (start 105.14 54.64) (end 101.905 54.64) (width 0.25) (layer "F.Cu") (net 27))
 (segment (start 108.5 63.31) (end 108.5 58) (width 0.25) (layer "F.Cu") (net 27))
 (segment (start 100.89 54.64) (end 101.905 54.64) (width 0.25) (layer "F.Cu") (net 27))
 (segment (start 100.61 53.64) (end 100.5 53.75) (width 0.25) (layer "F.Cu") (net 27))
 (segment (start 110 58.75) (end 105.39 54.14) (width 0.25) (layer "F.Cu") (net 26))
 (segment (start 105.39 54.14) (end 101.905 54.14) (width 0.25) (layer "F.Cu") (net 26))
 (segment (start 110 63.31) (end 110 58.75) (width 0.25) (layer "F.Cu") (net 26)))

